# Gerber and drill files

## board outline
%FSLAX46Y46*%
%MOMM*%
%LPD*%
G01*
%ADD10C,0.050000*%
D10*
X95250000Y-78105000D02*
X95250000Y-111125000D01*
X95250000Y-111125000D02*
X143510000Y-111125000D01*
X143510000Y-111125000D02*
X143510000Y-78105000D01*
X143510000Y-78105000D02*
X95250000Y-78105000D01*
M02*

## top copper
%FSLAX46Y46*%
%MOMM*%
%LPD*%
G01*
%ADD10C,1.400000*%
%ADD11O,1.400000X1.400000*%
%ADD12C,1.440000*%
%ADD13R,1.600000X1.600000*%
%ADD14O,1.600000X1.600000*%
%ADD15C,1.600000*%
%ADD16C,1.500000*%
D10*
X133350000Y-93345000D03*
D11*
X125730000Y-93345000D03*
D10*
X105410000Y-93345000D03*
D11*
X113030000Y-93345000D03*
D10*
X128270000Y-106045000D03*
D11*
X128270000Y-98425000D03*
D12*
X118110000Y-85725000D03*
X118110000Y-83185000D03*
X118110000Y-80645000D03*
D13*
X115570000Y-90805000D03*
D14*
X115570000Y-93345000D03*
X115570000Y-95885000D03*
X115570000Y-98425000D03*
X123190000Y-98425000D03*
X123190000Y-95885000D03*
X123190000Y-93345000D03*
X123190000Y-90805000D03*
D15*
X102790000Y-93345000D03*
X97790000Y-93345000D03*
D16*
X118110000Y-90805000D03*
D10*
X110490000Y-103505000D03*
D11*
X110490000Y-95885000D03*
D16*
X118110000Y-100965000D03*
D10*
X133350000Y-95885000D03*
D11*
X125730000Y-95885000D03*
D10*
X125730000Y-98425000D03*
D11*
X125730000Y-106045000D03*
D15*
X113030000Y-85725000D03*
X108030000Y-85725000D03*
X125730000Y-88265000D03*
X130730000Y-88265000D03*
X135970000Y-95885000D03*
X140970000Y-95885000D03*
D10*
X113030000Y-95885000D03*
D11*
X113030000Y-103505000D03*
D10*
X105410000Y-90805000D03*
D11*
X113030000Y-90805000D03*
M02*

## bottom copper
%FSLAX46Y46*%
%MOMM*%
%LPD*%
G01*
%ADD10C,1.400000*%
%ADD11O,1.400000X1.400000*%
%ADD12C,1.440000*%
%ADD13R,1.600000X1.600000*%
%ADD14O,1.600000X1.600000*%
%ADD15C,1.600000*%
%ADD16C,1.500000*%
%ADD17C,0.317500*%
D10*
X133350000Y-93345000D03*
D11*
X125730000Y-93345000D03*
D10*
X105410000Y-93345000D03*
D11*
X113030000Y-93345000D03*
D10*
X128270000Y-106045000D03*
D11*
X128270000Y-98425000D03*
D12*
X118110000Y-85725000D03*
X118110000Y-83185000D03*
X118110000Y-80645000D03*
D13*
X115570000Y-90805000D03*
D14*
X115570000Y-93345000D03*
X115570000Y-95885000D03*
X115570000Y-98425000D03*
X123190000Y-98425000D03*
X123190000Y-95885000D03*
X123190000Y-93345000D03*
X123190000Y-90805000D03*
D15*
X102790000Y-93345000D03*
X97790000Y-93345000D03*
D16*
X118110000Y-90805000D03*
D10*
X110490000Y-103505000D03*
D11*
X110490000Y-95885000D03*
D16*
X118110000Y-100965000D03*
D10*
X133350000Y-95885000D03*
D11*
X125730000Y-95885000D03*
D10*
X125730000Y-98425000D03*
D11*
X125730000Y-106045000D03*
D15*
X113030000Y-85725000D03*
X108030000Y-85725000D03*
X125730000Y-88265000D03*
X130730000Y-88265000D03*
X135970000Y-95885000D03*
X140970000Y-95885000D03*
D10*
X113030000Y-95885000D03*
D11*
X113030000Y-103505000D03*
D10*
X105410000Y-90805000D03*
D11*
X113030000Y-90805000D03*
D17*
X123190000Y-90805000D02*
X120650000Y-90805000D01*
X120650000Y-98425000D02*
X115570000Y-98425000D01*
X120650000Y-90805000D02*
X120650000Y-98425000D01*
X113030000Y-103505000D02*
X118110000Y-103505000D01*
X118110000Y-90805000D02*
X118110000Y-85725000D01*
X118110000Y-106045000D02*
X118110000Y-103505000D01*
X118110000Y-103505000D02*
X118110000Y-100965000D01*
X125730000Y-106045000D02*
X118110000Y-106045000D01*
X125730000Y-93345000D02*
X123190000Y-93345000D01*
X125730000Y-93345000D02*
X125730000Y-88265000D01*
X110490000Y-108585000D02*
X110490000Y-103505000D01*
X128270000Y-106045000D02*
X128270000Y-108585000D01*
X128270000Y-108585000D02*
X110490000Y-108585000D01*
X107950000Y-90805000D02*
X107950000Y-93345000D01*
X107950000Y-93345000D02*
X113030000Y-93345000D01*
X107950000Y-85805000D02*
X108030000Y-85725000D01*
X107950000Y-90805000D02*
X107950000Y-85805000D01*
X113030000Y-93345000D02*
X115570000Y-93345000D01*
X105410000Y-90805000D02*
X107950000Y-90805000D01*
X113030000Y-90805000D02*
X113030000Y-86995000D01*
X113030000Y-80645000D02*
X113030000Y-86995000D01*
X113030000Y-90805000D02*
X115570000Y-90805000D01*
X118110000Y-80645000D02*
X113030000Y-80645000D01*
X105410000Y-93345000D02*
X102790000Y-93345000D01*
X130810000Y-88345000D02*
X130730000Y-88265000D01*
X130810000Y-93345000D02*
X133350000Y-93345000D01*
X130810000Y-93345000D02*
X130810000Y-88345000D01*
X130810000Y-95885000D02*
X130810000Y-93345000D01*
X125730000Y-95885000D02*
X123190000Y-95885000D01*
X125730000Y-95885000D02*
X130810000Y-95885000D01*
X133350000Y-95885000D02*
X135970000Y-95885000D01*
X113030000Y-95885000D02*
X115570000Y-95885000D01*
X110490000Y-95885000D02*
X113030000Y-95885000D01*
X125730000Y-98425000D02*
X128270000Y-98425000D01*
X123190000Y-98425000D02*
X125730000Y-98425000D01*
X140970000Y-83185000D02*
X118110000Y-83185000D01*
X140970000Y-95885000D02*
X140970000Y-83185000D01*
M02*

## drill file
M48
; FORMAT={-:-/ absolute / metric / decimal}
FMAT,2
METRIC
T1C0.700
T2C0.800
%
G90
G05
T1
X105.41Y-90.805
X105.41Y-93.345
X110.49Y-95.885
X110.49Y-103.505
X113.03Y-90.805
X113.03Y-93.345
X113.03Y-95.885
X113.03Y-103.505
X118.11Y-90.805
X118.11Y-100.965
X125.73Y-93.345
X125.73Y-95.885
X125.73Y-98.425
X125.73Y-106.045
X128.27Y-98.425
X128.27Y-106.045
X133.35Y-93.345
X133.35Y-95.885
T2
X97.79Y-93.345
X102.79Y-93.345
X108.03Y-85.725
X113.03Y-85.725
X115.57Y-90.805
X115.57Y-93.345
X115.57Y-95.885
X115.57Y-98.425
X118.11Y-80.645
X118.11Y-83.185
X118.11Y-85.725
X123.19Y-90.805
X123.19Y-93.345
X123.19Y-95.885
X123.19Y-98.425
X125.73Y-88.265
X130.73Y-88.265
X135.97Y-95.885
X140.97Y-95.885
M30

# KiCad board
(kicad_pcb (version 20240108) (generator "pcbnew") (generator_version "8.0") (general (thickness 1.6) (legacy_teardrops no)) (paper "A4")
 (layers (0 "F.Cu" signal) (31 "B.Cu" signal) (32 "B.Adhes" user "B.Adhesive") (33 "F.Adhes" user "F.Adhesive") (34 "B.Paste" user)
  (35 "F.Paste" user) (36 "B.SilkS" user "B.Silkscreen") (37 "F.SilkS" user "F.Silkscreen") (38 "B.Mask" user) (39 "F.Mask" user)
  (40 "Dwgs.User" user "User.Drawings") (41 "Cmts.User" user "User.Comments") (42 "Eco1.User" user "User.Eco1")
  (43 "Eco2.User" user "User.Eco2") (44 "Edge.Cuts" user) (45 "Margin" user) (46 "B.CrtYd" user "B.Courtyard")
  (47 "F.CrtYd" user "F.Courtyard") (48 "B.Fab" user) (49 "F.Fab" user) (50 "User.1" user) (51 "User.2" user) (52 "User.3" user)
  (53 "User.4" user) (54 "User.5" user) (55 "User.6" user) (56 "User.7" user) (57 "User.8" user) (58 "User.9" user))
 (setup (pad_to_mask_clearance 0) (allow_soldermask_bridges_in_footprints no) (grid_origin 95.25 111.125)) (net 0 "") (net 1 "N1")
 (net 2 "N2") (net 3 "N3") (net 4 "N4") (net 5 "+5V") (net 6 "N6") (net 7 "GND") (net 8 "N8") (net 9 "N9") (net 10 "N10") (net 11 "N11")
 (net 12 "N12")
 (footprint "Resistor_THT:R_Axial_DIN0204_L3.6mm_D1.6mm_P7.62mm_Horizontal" (layer "F.Cu") (at 129.54 93.345 180)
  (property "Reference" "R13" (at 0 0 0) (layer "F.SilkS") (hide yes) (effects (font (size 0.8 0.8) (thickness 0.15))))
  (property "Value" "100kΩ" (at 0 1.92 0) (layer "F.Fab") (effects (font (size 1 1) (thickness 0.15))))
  (pad "1" thru_hole circle (at -3.81 0 180) (size 1.4 1.4) (drill 0.7) (layers "*.Cu" "*.Mask") (remove_unused_layers no) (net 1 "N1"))
  (pad "2" thru_hole oval (at 3.81 0 180) (size 1.4 1.4) (drill 0.7) (layers "*.Cu" "*.Mask") (remove_unused_layers no) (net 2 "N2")))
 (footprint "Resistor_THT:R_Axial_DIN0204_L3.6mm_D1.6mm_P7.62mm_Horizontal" (layer "F.Cu") (at 109.22 93.345)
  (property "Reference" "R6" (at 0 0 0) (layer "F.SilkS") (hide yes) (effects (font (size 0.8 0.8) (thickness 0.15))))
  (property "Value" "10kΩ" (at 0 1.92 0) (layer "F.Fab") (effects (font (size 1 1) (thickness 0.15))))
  (pad "1" thru_hole circle (at -3.81 0) (size 1.4 1.4) (drill 0.7) (layers "*.Cu" "*.Mask") (remove_unused_layers no) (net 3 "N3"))
  (pad "2" thru_hole oval (at 3.81 0) (size 1.4 1.4) (drill 0.7) (layers "*.Cu" "*.Mask") (remove_unused_layers no) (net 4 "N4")))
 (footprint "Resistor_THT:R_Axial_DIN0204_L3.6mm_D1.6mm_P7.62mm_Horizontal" (layer "F.Cu") (at 128.27 102.235 90)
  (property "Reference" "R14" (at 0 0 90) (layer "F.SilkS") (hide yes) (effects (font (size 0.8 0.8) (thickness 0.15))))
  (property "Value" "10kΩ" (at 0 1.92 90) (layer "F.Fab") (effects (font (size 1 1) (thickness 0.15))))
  (pad "1" thru_hole circle (at -3.81 0 90) (size 1.4 1.4) (drill 0.7) (layers "*.Cu" "*.Mask") (remove_unused_layers no) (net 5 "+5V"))
  (pad "2" thru_hole oval (at 3.81 0 90) (size 1.4 1.4) (drill 0.7) (layers "*.Cu" "*.Mask") (remove_unused_layers no) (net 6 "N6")))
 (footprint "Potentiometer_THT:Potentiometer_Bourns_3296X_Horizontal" (layer "F.Cu") (at 118.11 85.725 -90)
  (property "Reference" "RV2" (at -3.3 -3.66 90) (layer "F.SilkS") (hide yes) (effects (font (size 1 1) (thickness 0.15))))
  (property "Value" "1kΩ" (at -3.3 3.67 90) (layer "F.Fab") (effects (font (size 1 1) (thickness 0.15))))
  (pad "1" thru_hole circle (at 0 0 270) (size 1.44 1.44) (drill 0.8) (layers "*.Cu" "*.Mask") (remove_unused_layers no) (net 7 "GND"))
  (pad "2" thru_hole circle (at -2.54 0 270) (size 1.44 1.44) (drill 0.8) (layers "*.Cu" "*.Mask") (remove_unused_layers no) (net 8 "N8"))
  (pad "3" thru_hole circle (at -5.08 0 270) (size 1.44 1.44) (drill 0.8) (layers "*.Cu" "*.Mask") (remove_unused_layers no) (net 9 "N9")))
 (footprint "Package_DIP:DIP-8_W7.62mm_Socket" (layer "F.Cu") (at 119.38 94.615)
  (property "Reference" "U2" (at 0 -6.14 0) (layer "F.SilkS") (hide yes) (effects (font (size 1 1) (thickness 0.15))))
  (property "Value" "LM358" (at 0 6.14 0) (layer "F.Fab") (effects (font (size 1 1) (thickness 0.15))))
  (pad "1" thru_hole rect (at -3.81 -3.81) (size 1.6 1.6) (drill 0.8) (layers "*.Cu" "*.Mask") (remove_unused_layers no) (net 9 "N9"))
  (pad "2" thru_hole oval (at -3.81 -1.27) (size 1.6 1.6) (drill 0.8) (layers "*.Cu" "*.Mask") (remove_unused_layers no) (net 4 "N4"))
  (pad "3" thru_hole oval (at -3.81 1.27) (size 1.6 1.6) (drill 0.8) (layers "*.Cu" "*.Mask") (remove_unused_layers no) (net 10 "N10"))
  (pad "4" thru_hole oval (at -3.81 3.81) (size 1.6 1.6) (drill 0.8) (layers "*.Cu" "*.Mask") (remove_unused_layers no))
  (pad "5" thru_hole oval (at 3.81 3.81) (size 1.6 1.6) (drill 0.8) (layers "*.Cu" "*.Mask") (remove_unused_layers no) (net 6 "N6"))
  (pad "6" thru_hole oval (at 3.81 1.27) (size 1.6 1.6) (drill 0.8) (layers "*.Cu" "*.Mask") (remove_unused_layers no) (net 1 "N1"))
  (pad "7" thru_hole oval (at 3.81 -1.27) (size 1.6 1.6) (drill 0.8) (layers "*.Cu" "*.Mask") (remove_unused_layers no) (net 2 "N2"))
  (pad "8" thru_hole oval (at 3.81 -3.81) (size 1.6 1.6) (drill 0.8) (layers "*.Cu" "*.Mask") (remove_unused_layers no)))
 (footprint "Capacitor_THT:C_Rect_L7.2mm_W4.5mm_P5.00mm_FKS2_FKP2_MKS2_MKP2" (layer "F.Cu") (at 102.79 93.345 180)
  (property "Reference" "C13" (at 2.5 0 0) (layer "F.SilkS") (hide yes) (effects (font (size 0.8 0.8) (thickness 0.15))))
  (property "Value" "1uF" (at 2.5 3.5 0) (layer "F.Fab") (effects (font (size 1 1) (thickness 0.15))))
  (pad "1" thru_hole circle (at 0 0 180) (size 1.6 1.6) (drill 0.8) (layers "*.Cu" "*.Mask") (remove_unused_layers no) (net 3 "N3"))
  (pad "2" thru_hole circle (at 5 0 180) (size 1.6 1.6) (drill 0.8) (layers "*.Cu" "*.Mask") (remove_unused_layers no) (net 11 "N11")))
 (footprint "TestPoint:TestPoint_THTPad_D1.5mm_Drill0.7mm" (layer "F.Cu") (at 118.11 90.805)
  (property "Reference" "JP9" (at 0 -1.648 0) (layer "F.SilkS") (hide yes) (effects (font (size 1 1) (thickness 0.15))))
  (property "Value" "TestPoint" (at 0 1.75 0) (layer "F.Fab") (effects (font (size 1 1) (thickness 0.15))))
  (pad "1" thru_hole circle (at 0 0) (size 1.5 1.5) (drill 0.7) (layers "*.Cu" "*.Mask") (remove_unused_layers no) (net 7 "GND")))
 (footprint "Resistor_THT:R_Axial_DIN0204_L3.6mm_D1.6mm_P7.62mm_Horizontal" (layer "F.Cu") (at 110.49 99.695 90)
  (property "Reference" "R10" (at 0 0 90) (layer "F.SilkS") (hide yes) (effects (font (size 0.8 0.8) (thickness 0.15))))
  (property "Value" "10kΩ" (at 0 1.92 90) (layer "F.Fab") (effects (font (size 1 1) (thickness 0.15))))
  (pad "1" thru_hole circle (at -3.81 0 90) (size 1.4 1.4) (drill 0.7) (layers "*.Cu" "*.Mask") (remove_unused_layers no) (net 5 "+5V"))
  (pad "2" thru_hole oval (at 3.81 0 90) (size 1.4 1.4) (drill 0.7) (layers "*.Cu" "*.Mask") (remove_unused_layers no) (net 10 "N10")))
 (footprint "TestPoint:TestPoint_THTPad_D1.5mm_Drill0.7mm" (layer "F.Cu") (at 118.11 100.965)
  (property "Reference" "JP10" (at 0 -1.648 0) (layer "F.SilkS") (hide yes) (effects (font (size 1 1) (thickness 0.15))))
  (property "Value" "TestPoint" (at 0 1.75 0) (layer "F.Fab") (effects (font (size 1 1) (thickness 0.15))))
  (pad "1" thru_hole circle (at 0 0) (size 1.5 1.5) (drill 0.7) (layers "*.Cu" "*.Mask") (remove_unused_layers no) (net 7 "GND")))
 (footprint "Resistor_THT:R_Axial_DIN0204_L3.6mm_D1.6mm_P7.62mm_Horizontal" (layer "F.Cu") (at 129.54 95.885 180)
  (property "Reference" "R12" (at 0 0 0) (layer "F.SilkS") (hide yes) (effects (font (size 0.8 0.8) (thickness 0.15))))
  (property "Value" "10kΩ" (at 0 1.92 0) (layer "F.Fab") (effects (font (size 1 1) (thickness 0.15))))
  (pad "1" thru_hole circle (at -3.81 0 180) (size 1.4 1.4) (drill 0.7) (layers "*.Cu" "*.Mask") (remove_unused_layers no) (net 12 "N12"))
  (pad "2" thru_hole oval (at 3.81 0 180) (size 1.4 1.4) (drill 0.7) (layers "*.Cu" "*.Mask") (remove_unused_layers no) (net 1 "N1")))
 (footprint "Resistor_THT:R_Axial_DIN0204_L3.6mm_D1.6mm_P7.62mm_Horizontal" (layer "F.Cu") (at 125.73 102.235 -90)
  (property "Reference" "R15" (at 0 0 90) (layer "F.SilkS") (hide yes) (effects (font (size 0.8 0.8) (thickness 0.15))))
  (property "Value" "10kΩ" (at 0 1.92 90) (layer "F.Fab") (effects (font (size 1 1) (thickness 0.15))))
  (pad "1" thru_hole circle (at -3.81 0 270) (size 1.4 1.4) (drill 0.7) (layers "*.Cu" "*.Mask") (remove_unused_layers no) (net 6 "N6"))
  (pad "2" thru_hole oval (at 3.81 0 270) (size 1.4 1.4) (drill 0.7) (layers "*.Cu" "*.Mask") (remove_unused_layers no) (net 7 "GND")))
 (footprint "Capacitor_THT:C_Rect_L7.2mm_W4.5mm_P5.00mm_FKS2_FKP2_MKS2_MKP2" (layer "F.Cu") (at 113.03 85.725 180)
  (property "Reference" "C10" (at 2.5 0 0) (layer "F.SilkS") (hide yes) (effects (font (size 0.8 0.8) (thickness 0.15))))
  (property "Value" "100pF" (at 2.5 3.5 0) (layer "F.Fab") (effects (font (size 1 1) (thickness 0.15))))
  (pad "1" thru_hole circle (at 0 0 180) (size 1.6 1.6) (drill 0.8) (layers "*.Cu" "*.Mask") (remove_unused_layers no) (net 9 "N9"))
  (pad "2" thru_hole circle (at 5 0 180) (size 1.6 1.6) (drill 0.8) (layers "*.Cu" "*.Mask") (remove_unused_layers no) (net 4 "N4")))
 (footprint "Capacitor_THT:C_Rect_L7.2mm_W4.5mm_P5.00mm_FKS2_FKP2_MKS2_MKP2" (layer "F.Cu") (at 125.73 88.265)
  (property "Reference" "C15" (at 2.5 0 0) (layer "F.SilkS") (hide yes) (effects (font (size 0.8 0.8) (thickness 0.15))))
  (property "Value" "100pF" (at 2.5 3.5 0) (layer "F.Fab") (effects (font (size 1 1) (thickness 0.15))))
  (pad "1" thru_hole circle (at 0 0) (size 1.6 1.6) (drill 0.8) (layers "*.Cu" "*.Mask") (remove_unused_layers no) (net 2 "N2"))
  (pad "2" thru_hole circle (at 5 0) (size 1.6 1.6) (drill 0.8) (layers "*.Cu" "*.Mask") (remove_unused_layers no) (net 1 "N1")))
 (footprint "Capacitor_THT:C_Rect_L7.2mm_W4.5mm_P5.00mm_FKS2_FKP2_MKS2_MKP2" (layer "F.Cu") (at 135.97 95.885)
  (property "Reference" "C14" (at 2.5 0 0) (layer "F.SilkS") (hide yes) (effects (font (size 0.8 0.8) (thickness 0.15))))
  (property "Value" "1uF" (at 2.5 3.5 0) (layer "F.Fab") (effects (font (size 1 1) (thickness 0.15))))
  (pad "1" thru_hole circle (at 0 0) (size 1.6 1.6) (drill 0.8) (layers "*.Cu" "*.Mask") (remove_unused_layers no) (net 12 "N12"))
  (pad "2" thru_hole circle (at 5 0) (size 1.6 1.6) (drill 0.8) (layers "*.Cu" "*.Mask") (remove_unused_layers no) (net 8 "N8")))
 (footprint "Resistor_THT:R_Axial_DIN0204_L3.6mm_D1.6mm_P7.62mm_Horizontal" (layer "F.Cu") (at 113.03 99.695 -90)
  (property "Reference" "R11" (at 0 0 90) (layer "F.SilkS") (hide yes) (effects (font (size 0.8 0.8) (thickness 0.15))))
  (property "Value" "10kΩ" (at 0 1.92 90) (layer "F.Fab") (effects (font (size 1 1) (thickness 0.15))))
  (pad "1" thru_hole circle (at -3.81 0 270) (size 1.4 1.4) (drill 0.7) (layers "*.Cu" "*.Mask") (remove_unused_layers no) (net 10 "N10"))
  (pad "2" thru_hole oval (at 3.81 0 270) (size 1.4 1.4) (drill 0.7) (layers "*.Cu" "*.Mask") (remove_unused_layers no) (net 7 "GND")))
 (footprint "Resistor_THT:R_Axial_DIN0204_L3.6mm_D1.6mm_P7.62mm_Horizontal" (layer "F.Cu") (at 109.22 90.805)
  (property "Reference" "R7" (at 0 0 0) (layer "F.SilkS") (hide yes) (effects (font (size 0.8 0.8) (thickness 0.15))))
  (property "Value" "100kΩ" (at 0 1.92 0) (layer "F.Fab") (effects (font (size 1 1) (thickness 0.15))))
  (pad "1" thru_hole circle (at -3.81 0) (size 1.4 1.4) (drill 0.7) (layers "*.Cu" "*.Mask") (remove_unused_layers no) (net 4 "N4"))
  (pad "2" thru_hole oval (at 3.81 0) (size 1.4 1.4) (drill 0.7) (layers "*.Cu" "*.Mask") (remove_unused_layers no) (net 9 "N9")))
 (gr_line (start 95.25 78.105) (end 95.25 111.125) (stroke (width 0.05) (type default)) (layer "Edge.Cuts"))
 (gr_line (start 95.25 111.125) (end 143.51 111.125) (stroke (width 0.05) (type default)) (layer "Edge.Cuts"))
 (gr_line (start 143.51 111.125) (end 143.51 78.105) (stroke (width 0.05) (type default)) (layer "Edge.Cuts"))
 (gr_line (start 143.51 78.105) (end 95.25 78.105) (stroke (width 0.05) (type default)) (layer "Edge.Cuts"))
 (segment (start 123.19 90.805) (end 120.65 90.805) (width 0.3175) (layer "B.Cu") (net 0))
 (segment (start 120.65 98.425) (end 115.57 98.425) (width 0.3175) (layer "B.Cu") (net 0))
 (segment (start 120.65 90.805) (end 120.65 98.425) (width 0.3175) (layer "B.Cu") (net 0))
 (segment (start 113.03 103.505) (end 118.11 103.505) (width 0.3175) (layer "B.Cu") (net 7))
 (segment (start 118.11 90.805) (end 118.11 85.725) (width 0.3175) (layer "B.Cu") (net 7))
 (segment (start 118.11 106.045) (end 118.11 103.505) (width 0.3175) (layer "B.Cu") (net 7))
 (segment (start 118.11 103.505) (end 118.11 100.965) (width 0.3175) (layer "B.Cu") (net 7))
 (segment (start 125.73 106.045) (end 118.11 106.045) (width 0.3175) (layer "B.Cu") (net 7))
 (segment (start 125.73 93.345) (end 123.19 93.345) (width 0.3175) (layer "B.Cu") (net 2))
 (segment (start 125.73 93.345) (end 125.73 88.265) (width 0.3175) (layer "B.Cu") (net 2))
 (segment (start 110.49 108.585) (end 110.49 103.505) (width 0.3175) (layer "B.Cu") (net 5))
 (segment (start 128.27 106.045) (end 128.27 108.585) (width 0.3175) (layer "B.Cu") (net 5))
 (segment (start 128.27 108.585) (end 110.49 108.585) (width 0.3175) (layer "B.Cu") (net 5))
 (segment (start 107.95 90.805) (end 107.95 93.345) (width 0.3175) (layer "B.Cu") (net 4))
 (segment (start 107.95 93.345) (end 113.03 93.345) (width 0.3175) (layer "B.Cu") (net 4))
 (segment (start 107.95 85.805) (end 108.03 85.725) (width 0.3175) (layer "B.Cu") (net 4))
 (segment (start 107.95 90.805) (end 107.95 85.805) (width 0.3175) (layer "B.Cu") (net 4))
 (segment (start 113.03 93.345) (end 115.57 93.345) (width 0.3175) (layer "B.Cu") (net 4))
 (segment (start 105.41 90.805) (end 107.95 90.805) (width 0.3175) (layer "B.Cu") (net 4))
 (segment (start 113.03 90.805) (end 113.03 86.995) (width 0.3175) (layer "B.Cu") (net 9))
 (segment (start 113.03 80.645) (end 113.03 86.995) (width 0.3175) (layer "B.Cu") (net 9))
 (segment (start 113.03 90.805) (end 115.57 90.805) (width 0.3175) (layer "B.Cu") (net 9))
 (segment (start 118.11 80.645) (end 113.03 80.645) (width 0.3175) (layer "B.Cu") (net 9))
 (segment (start 105.41 93.345) (end 102.79 93.345) (width 0.3175) (layer "B.Cu") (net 3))
 (segment (start 130.81 88.345) (end 130.73 88.265) (width 0.3175) (layer "B.Cu") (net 1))
 (segment (start 130.81 93.345) (end 133.35 93.345) (width 0.3175) (layer "B.Cu") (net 1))
 (segment (start 130.81 93.345) (end 130.81 88.345) (width 0.3175) (layer "B.Cu") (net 1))
 (segment (start 130.81 95.885) (end 130.81 93.345) (width 0.3175) (layer "B.Cu") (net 1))
 (segment (start 125.73 95.885) (end 123.19 95.885) (width 0.3175) (layer "B.Cu") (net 1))
 (segment (start 125.73 95.885) (end 130.81 95.885) (width 0.3175) (layer "B.Cu") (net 1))
 (segment (start 133.35 95.885) (end 135.97 95.885) (width 0.3175) (layer "B.Cu") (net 12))
 (segment (start 113.03 95.885) (end 115.57 95.885) (width 0.3175) (layer "B.Cu") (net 10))
 (segment (start 110.49 95.885) (end 113.03 95.885) (width 0.3175) (layer "B.Cu") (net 10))
 (segment (start 125.73 98.425) (end 128.27 98.425) (width 0.3175) (layer "B.Cu") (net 6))
 (segment (start 123.19 98.425) (end 125.73 98.425) (width 0.3175) (layer "B.Cu") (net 6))
 (segment (start 140.97 83.185) (end 118.11 83.185) (width 0.3175) (layer "B.Cu") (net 8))
 (segment (start 140.97 95.885) (end 140.97 83.185) (width 0.3175) (layer "B.Cu") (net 8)))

